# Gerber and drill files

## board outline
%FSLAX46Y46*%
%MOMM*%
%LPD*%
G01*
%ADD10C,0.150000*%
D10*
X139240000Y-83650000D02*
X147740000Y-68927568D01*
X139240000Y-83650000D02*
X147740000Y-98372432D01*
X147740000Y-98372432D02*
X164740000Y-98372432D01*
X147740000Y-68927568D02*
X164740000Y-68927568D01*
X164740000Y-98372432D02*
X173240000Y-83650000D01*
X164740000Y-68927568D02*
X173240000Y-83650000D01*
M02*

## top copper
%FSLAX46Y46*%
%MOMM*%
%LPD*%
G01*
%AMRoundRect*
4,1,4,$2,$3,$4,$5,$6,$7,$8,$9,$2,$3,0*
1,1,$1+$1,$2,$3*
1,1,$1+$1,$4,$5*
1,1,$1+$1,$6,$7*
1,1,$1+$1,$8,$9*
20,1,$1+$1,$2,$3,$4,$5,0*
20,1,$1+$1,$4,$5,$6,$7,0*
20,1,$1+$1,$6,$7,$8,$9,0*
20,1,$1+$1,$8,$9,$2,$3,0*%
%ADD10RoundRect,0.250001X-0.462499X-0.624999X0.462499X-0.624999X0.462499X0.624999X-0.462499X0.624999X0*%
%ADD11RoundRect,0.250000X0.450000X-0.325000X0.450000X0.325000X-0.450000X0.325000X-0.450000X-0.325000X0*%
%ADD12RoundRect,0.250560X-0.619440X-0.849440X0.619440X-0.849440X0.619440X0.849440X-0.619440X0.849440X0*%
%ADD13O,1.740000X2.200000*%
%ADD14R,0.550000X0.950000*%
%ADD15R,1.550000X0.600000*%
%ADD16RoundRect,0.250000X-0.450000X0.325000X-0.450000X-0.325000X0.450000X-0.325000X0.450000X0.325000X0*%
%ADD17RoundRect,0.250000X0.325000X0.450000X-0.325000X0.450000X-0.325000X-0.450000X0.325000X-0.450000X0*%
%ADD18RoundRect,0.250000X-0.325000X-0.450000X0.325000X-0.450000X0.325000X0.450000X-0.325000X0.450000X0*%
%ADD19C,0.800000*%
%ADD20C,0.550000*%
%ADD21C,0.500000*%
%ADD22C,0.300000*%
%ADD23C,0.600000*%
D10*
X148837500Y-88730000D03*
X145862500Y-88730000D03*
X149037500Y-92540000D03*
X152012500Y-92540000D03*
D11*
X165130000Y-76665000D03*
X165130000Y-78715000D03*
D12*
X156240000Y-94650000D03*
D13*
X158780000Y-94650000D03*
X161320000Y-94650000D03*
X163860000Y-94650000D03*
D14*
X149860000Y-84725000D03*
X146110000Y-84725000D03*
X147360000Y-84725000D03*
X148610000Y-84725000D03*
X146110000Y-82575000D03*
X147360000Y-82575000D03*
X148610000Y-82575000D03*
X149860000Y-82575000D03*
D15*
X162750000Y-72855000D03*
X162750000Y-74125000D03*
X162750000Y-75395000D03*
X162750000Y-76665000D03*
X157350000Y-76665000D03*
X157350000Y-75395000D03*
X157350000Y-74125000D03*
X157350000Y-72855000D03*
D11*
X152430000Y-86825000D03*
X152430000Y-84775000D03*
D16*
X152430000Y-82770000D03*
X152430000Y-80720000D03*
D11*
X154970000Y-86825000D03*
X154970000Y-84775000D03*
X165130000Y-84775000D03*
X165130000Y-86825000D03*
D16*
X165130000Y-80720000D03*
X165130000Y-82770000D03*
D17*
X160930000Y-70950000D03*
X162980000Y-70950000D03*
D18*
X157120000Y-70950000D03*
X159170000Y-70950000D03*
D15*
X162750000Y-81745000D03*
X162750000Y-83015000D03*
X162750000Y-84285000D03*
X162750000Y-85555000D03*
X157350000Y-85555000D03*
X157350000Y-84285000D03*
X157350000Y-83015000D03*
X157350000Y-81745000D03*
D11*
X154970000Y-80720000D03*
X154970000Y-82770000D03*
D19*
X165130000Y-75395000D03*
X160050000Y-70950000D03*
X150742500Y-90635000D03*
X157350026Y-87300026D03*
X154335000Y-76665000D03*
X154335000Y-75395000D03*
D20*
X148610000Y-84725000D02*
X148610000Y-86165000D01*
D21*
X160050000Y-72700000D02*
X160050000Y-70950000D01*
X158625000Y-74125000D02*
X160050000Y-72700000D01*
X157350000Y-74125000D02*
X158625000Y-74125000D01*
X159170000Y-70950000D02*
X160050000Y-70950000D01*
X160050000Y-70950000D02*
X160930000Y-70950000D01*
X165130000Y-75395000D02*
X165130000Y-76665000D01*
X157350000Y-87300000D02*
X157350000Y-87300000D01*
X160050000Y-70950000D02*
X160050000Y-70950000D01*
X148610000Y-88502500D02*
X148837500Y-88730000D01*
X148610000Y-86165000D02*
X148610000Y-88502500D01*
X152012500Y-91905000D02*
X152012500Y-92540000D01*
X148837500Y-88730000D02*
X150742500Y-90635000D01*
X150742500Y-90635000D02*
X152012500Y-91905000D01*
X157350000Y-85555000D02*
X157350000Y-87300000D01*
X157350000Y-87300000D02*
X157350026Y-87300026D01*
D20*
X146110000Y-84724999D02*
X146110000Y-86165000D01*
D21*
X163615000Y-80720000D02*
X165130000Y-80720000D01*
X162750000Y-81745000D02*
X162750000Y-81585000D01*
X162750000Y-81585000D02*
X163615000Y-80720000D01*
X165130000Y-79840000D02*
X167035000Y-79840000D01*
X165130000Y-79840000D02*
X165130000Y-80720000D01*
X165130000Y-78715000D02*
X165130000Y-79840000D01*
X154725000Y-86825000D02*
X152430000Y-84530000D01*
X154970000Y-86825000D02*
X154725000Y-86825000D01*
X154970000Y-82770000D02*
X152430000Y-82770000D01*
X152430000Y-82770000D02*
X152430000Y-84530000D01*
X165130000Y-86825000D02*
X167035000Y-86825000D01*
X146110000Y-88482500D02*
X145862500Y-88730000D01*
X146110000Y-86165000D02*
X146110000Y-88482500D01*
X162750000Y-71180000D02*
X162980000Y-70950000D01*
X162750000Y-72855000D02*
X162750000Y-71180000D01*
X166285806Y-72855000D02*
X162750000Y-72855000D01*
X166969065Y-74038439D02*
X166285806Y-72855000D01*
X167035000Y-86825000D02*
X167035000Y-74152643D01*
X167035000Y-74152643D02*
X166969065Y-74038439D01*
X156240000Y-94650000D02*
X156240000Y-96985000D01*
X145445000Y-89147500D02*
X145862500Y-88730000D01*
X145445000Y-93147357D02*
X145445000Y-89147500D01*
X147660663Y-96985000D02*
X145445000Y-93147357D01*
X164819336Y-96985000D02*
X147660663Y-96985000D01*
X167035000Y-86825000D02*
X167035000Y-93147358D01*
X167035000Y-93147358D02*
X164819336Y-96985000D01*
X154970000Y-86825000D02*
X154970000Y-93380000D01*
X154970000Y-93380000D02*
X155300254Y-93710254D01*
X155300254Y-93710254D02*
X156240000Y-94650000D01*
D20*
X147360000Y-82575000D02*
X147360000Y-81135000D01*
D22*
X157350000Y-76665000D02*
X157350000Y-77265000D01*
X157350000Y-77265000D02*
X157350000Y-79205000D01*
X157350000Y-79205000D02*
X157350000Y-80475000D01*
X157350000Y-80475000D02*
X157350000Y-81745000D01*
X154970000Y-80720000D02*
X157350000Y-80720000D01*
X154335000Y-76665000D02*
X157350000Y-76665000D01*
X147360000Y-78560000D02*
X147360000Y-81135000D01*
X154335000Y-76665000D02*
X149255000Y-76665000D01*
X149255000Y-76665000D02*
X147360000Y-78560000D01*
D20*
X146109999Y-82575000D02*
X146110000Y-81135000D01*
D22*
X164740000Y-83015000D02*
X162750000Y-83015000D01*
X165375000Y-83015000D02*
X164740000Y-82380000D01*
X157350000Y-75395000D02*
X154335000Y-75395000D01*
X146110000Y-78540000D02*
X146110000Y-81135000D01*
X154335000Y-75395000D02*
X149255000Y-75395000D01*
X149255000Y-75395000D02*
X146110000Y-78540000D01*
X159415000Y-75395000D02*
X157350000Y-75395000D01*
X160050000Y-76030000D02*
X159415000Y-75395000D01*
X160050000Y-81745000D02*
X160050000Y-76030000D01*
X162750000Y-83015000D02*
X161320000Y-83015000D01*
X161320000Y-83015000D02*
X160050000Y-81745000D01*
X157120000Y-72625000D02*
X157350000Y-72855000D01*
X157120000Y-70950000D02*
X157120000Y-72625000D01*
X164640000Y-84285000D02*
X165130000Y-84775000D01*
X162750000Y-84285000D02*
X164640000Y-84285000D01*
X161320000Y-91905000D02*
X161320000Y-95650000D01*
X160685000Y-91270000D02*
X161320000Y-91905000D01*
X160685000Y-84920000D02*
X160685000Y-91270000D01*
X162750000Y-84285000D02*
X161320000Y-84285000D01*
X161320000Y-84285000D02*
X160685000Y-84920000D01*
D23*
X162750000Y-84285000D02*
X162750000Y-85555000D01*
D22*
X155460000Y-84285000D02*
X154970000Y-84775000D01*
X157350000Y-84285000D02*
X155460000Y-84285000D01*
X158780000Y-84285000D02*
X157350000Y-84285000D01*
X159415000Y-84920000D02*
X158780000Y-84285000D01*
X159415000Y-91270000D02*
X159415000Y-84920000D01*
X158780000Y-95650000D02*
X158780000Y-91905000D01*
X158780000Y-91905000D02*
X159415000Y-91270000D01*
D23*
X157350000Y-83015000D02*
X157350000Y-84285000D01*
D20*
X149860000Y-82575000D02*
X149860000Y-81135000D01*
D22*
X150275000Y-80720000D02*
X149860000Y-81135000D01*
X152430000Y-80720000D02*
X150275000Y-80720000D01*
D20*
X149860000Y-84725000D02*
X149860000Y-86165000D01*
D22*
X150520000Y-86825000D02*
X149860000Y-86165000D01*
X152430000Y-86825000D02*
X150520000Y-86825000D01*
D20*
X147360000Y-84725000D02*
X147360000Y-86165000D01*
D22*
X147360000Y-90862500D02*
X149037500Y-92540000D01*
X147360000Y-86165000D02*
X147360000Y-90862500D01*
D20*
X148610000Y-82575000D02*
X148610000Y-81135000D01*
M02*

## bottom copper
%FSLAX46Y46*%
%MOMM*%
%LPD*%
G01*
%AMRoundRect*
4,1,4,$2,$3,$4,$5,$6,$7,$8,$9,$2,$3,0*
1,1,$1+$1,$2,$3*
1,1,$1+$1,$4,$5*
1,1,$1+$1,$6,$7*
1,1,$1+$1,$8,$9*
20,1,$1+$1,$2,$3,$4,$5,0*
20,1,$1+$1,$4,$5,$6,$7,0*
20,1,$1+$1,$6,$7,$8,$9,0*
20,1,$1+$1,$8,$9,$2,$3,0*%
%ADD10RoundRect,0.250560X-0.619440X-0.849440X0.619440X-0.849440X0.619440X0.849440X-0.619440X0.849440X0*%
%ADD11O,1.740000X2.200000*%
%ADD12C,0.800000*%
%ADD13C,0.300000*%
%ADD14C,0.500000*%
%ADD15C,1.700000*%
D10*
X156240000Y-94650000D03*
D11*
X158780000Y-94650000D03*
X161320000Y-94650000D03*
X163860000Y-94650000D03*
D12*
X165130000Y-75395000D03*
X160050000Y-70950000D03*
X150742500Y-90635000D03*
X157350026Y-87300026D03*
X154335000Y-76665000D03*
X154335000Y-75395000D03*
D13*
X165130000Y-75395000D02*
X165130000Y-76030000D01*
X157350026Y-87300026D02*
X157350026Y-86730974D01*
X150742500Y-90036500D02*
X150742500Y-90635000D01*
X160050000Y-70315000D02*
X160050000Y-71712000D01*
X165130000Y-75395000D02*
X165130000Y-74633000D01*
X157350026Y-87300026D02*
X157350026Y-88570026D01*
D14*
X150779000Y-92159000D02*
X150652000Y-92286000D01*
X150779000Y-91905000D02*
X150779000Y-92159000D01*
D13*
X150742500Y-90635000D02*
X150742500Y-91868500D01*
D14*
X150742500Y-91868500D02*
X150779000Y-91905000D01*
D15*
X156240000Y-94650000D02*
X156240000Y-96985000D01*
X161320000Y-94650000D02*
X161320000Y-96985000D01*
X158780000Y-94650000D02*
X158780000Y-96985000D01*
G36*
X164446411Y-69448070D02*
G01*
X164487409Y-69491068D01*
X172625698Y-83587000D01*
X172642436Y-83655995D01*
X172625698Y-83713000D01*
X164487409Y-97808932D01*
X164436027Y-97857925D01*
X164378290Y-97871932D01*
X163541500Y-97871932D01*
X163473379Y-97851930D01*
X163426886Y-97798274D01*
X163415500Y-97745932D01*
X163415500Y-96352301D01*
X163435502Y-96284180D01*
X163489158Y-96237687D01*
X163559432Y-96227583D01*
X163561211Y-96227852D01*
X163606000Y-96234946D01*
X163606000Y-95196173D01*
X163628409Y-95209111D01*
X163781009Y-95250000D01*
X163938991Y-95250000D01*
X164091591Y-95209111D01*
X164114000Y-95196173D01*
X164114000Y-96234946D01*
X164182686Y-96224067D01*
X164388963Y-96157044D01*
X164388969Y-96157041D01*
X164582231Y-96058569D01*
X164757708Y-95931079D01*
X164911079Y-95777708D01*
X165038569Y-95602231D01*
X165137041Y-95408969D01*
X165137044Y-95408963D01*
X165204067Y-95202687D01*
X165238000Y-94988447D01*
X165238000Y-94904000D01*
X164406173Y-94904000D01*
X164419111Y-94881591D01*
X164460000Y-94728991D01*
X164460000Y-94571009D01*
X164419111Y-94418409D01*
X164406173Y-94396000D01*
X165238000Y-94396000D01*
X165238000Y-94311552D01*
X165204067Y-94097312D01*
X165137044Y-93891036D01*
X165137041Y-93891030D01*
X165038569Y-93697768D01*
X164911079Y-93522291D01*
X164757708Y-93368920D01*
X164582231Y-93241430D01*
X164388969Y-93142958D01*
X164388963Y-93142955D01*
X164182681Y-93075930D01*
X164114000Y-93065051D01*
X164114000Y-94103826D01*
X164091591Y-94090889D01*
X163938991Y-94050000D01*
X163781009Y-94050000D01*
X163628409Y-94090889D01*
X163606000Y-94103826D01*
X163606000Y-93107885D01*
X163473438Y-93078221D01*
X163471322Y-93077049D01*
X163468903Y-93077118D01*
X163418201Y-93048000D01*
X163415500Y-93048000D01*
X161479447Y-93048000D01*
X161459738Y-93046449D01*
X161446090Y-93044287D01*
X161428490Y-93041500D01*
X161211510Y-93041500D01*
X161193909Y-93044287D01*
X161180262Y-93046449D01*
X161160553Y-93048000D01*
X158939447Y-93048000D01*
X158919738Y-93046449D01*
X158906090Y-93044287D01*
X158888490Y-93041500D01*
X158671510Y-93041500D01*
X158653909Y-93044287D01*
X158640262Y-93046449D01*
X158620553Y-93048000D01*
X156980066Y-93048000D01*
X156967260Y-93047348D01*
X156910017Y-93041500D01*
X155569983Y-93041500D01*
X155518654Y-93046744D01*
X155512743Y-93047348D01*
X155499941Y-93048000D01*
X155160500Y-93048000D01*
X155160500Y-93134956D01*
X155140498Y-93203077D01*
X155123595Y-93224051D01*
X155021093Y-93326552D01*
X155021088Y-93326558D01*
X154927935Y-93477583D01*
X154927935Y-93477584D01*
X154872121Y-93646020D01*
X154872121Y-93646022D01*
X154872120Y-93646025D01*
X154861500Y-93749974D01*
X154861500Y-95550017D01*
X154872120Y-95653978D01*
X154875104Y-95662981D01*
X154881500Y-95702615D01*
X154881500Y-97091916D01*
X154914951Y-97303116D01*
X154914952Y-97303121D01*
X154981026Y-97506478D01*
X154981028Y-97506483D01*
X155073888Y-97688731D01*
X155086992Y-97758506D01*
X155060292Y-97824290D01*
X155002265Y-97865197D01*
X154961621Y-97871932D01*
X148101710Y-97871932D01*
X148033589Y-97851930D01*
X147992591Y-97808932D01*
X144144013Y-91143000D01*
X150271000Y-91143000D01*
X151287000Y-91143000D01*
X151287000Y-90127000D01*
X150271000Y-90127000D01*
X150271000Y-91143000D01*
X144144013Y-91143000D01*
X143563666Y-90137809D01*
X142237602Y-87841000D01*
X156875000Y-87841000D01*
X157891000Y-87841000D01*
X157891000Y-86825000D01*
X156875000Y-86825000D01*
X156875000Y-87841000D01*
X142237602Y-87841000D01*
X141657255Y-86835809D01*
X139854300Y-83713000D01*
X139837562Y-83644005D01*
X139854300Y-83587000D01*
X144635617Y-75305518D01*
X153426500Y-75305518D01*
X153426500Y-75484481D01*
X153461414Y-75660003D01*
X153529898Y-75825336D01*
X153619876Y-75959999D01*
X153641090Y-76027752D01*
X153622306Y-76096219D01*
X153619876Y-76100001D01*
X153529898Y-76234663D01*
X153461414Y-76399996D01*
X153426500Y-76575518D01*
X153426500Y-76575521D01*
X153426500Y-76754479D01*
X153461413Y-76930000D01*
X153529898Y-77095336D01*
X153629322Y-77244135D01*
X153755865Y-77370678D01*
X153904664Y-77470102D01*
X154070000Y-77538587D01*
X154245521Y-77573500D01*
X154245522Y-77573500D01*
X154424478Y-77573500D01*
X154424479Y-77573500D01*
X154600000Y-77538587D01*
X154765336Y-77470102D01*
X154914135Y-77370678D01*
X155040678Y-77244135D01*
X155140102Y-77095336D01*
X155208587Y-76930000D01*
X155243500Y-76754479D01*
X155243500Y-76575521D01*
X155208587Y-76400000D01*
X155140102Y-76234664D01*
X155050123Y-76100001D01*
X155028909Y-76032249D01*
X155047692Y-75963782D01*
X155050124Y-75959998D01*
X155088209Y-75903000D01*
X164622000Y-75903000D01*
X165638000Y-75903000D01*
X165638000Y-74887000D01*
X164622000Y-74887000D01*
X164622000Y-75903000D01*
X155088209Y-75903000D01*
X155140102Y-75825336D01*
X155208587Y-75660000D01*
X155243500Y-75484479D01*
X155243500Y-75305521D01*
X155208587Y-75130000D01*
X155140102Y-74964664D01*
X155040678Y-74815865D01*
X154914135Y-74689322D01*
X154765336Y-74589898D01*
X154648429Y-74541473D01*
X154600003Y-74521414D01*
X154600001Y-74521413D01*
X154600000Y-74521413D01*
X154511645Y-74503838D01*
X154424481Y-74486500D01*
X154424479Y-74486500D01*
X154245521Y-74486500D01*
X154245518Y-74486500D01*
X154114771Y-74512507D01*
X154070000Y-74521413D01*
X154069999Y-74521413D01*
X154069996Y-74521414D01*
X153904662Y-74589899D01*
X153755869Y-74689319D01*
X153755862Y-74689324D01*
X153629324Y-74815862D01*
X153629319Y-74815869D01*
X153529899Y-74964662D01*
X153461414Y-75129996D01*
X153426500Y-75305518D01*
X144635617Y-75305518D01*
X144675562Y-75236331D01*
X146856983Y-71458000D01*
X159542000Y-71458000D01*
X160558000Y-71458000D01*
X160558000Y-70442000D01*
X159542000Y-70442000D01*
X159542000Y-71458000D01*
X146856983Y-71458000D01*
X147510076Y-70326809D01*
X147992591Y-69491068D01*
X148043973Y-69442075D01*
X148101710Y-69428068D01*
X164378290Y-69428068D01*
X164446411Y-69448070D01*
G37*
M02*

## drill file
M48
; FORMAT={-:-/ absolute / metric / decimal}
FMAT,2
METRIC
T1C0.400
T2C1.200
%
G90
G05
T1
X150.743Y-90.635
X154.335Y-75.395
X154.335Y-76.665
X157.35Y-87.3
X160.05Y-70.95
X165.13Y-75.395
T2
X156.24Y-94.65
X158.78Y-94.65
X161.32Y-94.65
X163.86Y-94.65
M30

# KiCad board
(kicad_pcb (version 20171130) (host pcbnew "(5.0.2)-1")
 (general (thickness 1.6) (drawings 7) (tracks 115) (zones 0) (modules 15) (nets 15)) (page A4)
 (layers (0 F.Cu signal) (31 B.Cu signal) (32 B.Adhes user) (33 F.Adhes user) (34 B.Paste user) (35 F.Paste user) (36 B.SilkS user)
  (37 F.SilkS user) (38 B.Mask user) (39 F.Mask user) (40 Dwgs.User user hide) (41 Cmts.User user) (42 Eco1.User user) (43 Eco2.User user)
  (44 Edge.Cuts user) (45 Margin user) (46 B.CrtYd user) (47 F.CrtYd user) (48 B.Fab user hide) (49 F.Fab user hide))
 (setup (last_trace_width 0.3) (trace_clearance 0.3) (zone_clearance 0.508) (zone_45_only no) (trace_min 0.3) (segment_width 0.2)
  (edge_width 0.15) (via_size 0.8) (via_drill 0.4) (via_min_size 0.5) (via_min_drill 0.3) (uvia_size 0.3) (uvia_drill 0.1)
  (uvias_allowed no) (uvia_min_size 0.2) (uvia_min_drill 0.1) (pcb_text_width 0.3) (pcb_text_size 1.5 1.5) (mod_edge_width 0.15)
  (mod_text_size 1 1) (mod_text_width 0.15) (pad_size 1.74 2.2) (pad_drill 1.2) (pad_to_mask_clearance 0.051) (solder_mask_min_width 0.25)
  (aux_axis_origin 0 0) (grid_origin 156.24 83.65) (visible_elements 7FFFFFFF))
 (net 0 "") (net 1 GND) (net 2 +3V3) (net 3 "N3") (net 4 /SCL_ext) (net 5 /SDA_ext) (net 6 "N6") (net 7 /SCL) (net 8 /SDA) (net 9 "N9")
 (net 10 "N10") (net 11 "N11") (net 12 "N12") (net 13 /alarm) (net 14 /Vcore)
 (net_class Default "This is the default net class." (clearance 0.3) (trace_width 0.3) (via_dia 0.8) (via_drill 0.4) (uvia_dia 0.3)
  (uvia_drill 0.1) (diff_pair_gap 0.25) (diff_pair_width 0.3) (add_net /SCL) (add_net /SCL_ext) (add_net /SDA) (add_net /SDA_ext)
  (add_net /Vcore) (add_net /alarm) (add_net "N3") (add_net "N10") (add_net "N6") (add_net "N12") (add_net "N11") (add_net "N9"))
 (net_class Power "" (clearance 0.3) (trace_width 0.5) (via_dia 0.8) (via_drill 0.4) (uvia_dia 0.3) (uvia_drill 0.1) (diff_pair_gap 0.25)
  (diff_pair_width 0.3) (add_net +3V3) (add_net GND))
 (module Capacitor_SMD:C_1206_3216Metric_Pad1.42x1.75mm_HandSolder (layer F.Cu) (at 147.35 88.73)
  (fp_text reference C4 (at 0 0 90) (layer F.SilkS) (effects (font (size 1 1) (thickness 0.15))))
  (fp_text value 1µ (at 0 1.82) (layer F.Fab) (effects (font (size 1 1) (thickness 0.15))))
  (pad 2 smd roundrect (at 1.4875 0) (size 1.425 1.75) (layers F.Cu F.Paste F.Mask) (roundrect_rratio 0.175439) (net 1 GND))
  (pad 1 smd roundrect (at -1.4875 0) (size 1.425 1.75) (layers F.Cu F.Paste F.Mask) (roundrect_rratio 0.175439) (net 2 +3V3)))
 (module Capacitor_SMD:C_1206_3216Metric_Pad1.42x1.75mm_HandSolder (layer F.Cu) (at 150.525 92.54)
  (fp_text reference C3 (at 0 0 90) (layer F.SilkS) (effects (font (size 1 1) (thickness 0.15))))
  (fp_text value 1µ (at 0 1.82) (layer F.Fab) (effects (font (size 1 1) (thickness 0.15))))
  (pad 1 smd roundrect (at -1.4875 0) (size 1.425 1.75) (layers F.Cu F.Paste F.Mask) (roundrect_rratio 0.175439) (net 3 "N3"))
  (pad 2 smd roundrect (at 1.4875 0) (size 1.425 1.75) (layers F.Cu F.Paste F.Mask) (roundrect_rratio 0.175439) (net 1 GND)))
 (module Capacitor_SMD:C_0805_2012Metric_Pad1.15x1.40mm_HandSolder (layer F.Cu) (at 165.13 77.69 90)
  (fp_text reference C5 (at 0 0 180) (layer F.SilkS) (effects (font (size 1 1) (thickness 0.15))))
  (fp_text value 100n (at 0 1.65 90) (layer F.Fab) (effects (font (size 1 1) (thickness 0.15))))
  (pad 2 smd roundrect (at 1.025 0 90) (size 1.15 1.4) (layers F.Cu F.Paste F.Mask) (roundrect_rratio 0.217391) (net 1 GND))
  (pad 1 smd roundrect (at -1.025 0 90) (size 1.15 1.4) (layers F.Cu F.Paste F.Mask) (roundrect_rratio 0.217391) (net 2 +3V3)))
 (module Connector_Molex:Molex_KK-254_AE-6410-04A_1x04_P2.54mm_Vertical (layer F.Cu) (at 156.24 94.65)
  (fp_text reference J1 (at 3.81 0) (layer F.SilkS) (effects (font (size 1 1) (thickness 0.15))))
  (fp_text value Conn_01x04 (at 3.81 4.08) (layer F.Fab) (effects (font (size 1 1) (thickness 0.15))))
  (pad 1 thru_hole roundrect (at 0 0) (size 1.74 2.2) (drill 1.2) (layers *.Cu *.Mask) (roundrect_rratio 0.144) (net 2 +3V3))
  (pad 2 thru_hole oval (at 2.54 0) (size 1.74 2.2) (drill 1.2) (layers *.Cu *.Mask) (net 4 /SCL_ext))
  (pad 3 thru_hole oval (at 5.08 0) (size 1.74 2.2) (drill 1.2) (layers *.Cu *.Mask) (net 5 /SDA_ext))
  (pad 4 thru_hole oval (at 7.62 0) (size 1.74 2.2) (drill 1.2) (layers *.Cu *.Mask) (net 1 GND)))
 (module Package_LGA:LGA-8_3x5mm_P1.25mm (layer F.Cu) (at 147.985 83.65 90)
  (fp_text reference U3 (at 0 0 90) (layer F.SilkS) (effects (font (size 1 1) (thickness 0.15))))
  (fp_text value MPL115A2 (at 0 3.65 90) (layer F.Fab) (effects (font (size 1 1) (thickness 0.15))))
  (pad 4 smd rect (at -1.075 1.875 90) (size 0.95 0.55) (layers F.Cu F.Paste F.Mask) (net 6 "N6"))
  (pad 1 smd rect (at -1.075 -1.875 90) (size 0.95 0.55) (layers F.Cu F.Paste F.Mask) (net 2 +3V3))
  (pad 2 smd rect (at -1.075 -0.625 90) (size 0.95 0.55) (layers F.Cu F.Paste F.Mask) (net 3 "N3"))
  (pad 3 smd rect (at -1.075 0.625 90) (size 0.95 0.55) (layers F.Cu F.Paste F.Mask) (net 1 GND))
  (pad 8 smd rect (at 1.075 -1.875 90) (size 0.95 0.55) (layers F.Cu F.Paste F.Mask) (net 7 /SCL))
  (pad 7 smd rect (at 1.075 -0.625 90) (size 0.95 0.55) (layers F.Cu F.Paste F.Mask) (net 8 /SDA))
  (pad 6 smd rect (at 1.075 0.625 90) (size 0.95 0.55) (layers F.Cu F.Paste F.Mask) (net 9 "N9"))
  (pad 5 smd rect (at 1.075 1.875 90) (size 0.95 0.55) (layers F.Cu F.Paste F.Mask) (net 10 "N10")))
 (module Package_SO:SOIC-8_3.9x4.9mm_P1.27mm (layer F.Cu) (at 160.05 74.76)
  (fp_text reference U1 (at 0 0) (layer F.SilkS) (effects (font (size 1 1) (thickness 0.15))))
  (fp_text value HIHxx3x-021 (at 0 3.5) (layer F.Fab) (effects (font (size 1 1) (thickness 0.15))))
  (pad 8 smd rect (at 2.7 -1.905) (size 1.55 0.6) (layers F.Cu F.Paste F.Mask) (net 2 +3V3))
  (pad 7 smd rect (at 2.7 -0.635) (size 1.55 0.6) (layers F.Cu F.Paste F.Mask) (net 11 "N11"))
  (pad 6 smd rect (at 2.7 0.635) (size 1.55 0.6) (layers F.Cu F.Paste F.Mask) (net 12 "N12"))
  (pad 5 smd rect (at 2.7 1.905) (size 1.55 0.6) (layers F.Cu F.Paste F.Mask) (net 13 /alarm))
  (pad 4 smd rect (at -2.7 1.905) (size 1.55 0.6) (layers F.Cu F.Paste F.Mask) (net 8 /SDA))
  (pad 3 smd rect (at -2.7 0.635) (size 1.55 0.6) (layers F.Cu F.Paste F.Mask) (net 7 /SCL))
  (pad 2 smd rect (at -2.7 -0.635) (size 1.55 0.6) (layers F.Cu F.Paste F.Mask) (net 1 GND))
  (pad 1 smd rect (at -2.7 -1.905) (size 1.55 0.6) (layers F.Cu F.Paste F.Mask) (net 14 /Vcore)))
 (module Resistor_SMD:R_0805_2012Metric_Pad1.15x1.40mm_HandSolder (layer F.Cu) (at 152.43 85.8 90)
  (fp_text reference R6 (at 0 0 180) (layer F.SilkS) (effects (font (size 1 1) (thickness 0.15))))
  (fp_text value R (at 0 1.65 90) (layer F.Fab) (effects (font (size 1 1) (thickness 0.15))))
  (pad 1 smd roundrect (at -1.025 0 90) (size 1.15 1.4) (layers F.Cu F.Paste F.Mask) (roundrect_rratio 0.217391) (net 6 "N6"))
  (pad 2 smd roundrect (at 1.025 0 90) (size 1.15 1.4) (layers F.Cu F.Paste F.Mask) (roundrect_rratio 0.217391) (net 2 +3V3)))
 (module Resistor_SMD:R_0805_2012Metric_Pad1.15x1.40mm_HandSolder (layer F.Cu) (at 152.43 81.745 270)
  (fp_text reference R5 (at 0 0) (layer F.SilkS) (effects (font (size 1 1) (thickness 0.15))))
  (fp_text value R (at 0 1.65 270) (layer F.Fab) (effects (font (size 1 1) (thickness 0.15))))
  (pad 2 smd roundrect (at 1.025 0 270) (size 1.15 1.4) (layers F.Cu F.Paste F.Mask) (roundrect_rratio 0.217391) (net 2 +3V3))
  (pad 1 smd roundrect (at -1.025 0 270) (size 1.15 1.4) (layers F.Cu F.Paste F.Mask) (roundrect_rratio 0.217391) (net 10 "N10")))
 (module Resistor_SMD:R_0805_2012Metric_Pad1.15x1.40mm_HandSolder (layer F.Cu) (at 154.97 85.8 90)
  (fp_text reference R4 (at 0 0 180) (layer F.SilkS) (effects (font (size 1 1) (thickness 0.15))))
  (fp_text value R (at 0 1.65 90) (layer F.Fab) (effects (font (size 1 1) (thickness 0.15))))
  (pad 1 smd roundrect (at -1.025 0 90) (size 1.15 1.4) (layers F.Cu F.Paste F.Mask) (roundrect_rratio 0.217391) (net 2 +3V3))
  (pad 2 smd roundrect (at 1.025 0 90) (size 1.15 1.4) (layers F.Cu F.Paste F.Mask) (roundrect_rratio 0.217391) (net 4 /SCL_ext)))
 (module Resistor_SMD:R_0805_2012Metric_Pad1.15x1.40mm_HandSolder (layer F.Cu) (at 165.13 85.8 90)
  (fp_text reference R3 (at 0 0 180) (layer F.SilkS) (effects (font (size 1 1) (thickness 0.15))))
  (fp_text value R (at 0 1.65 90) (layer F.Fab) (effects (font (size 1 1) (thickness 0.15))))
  (pad 2 smd roundrect (at 1.025 0 90) (size 1.15 1.4) (layers F.Cu F.Paste F.Mask) (roundrect_rratio 0.217391) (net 5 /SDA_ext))
  (pad 1 smd roundrect (at -1.025 0 90) (size 1.15 1.4) (layers F.Cu F.Paste F.Mask) (roundrect_rratio 0.217391) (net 2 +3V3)))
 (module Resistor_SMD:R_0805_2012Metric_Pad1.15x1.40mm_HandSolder (layer F.Cu) (at 165.13 81.745 270)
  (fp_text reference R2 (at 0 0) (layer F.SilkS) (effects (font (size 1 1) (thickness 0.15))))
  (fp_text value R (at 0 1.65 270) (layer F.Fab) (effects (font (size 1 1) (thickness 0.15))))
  (pad 1 smd roundrect (at -1.025 0 270) (size 1.15 1.4) (layers F.Cu F.Paste F.Mask) (roundrect_rratio 0.217391) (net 2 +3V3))
  (pad 2 smd roundrect (at 1.025 0 270) (size 1.15 1.4) (layers F.Cu F.Paste F.Mask) (roundrect_rratio 0.217391) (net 7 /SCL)))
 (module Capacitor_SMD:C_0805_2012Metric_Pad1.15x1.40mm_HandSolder (layer F.Cu) (at 161.955 70.95 180)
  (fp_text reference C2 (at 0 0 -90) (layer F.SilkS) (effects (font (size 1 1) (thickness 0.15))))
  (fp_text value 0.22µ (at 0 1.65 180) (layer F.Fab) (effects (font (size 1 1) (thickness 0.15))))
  (pad 2 smd roundrect (at 1.025 0 180) (size 1.15 1.4) (layers F.Cu F.Paste F.Mask) (roundrect_rratio 0.217391) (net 1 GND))
  (pad 1 smd roundrect (at -1.025 0 180) (size 1.15 1.4) (layers F.Cu F.Paste F.Mask) (roundrect_rratio 0.217391) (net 2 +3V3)))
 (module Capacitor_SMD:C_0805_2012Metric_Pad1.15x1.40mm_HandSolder (layer F.Cu) (at 158.145 70.95)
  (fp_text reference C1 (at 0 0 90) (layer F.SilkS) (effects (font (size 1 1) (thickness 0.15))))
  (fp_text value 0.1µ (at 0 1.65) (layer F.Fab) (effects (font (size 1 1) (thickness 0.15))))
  (pad 1 smd roundrect (at -1.025 0) (size 1.15 1.4) (layers F.Cu F.Paste F.Mask) (roundrect_rratio 0.217391) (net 14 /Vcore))
  (pad 2 smd roundrect (at 1.025 0) (size 1.15 1.4) (layers F.Cu F.Paste F.Mask) (roundrect_rratio 0.217391) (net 1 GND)))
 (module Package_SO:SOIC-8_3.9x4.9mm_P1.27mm (layer F.Cu) (at 160.05 83.65)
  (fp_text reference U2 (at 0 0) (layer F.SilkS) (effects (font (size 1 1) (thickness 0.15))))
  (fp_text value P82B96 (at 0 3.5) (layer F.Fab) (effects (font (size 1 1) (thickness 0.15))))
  (pad 8 smd rect (at 2.7 -1.905) (size 1.55 0.6) (layers F.Cu F.Paste F.Mask) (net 2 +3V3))
  (pad 7 smd rect (at 2.7 -0.635) (size 1.55 0.6) (layers F.Cu F.Paste F.Mask) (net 7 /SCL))
  (pad 6 smd rect (at 2.7 0.635) (size 1.55 0.6) (layers F.Cu F.Paste F.Mask) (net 5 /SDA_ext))
  (pad 5 smd rect (at 2.7 1.905) (size 1.55 0.6) (layers F.Cu F.Paste F.Mask) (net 5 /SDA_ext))
  (pad 4 smd rect (at -2.7 1.905) (size 1.55 0.6) (layers F.Cu F.Paste F.Mask) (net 1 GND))
  (pad 3 smd rect (at -2.7 0.635) (size 1.55 0.6) (layers F.Cu F.Paste F.Mask) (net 4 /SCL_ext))
  (pad 2 smd rect (at -2.7 -0.635) (size 1.55 0.6) (layers F.Cu F.Paste F.Mask) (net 4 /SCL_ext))
  (pad 1 smd rect (at -2.7 -1.905) (size 1.55 0.6) (layers F.Cu F.Paste F.Mask) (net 8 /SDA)))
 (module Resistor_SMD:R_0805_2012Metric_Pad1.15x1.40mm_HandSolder (layer F.Cu) (at 154.97 81.745 90)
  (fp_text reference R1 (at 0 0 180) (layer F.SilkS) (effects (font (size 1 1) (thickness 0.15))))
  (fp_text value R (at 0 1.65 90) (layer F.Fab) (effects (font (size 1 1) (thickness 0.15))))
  (pad 2 smd roundrect (at 1.025 0 90) (size 1.15 1.4) (layers F.Cu F.Paste F.Mask) (roundrect_rratio 0.217391) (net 8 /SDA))
  (pad 1 smd roundrect (at -1.025 0 90) (size 1.15 1.4) (layers F.Cu F.Paste F.Mask) (roundrect_rratio 0.217391) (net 2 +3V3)))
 (gr_line (start 139.24 83.65) (end 147.74 68.927568) (layer Edge.Cuts) (width 0.15))
 (gr_line (start 139.24 83.65) (end 147.74 98.372432) (layer Edge.Cuts) (width 0.15))
 (gr_line (start 147.74 98.372432) (end 164.74 98.372432) (layer Edge.Cuts) (width 0.15))
 (gr_line (start 147.74 68.927568) (end 164.74 68.927568) (layer Edge.Cuts) (width 0.15))
 (gr_line (start 164.74 98.372432) (end 173.24 83.65) (layer Edge.Cuts) (width 0.15))
 (gr_line (start 164.74 68.927568) (end 173.24 83.65) (layer Edge.Cuts) (width 0.15))
 (segment (start 148.61 84.725) (end 148.61 86.165) (width 0.55) (layer F.Cu) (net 1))
 (segment (start 160.05 72.7) (end 160.05 70.95) (width 0.5) (layer F.Cu) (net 1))
 (segment (start 158.625 74.125) (end 160.05 72.7) (width 0.5) (layer F.Cu) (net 1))
 (segment (start 157.35 74.125) (end 158.625 74.125) (width 0.5) (layer F.Cu) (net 1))
 (segment (start 159.17 70.95) (end 160.05 70.95) (width 0.5) (layer F.Cu) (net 1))
 (segment (start 160.05 70.95) (end 160.93 70.95) (width 0.5) (layer F.Cu) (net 1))
 (via (at 165.13 75.395) (size 0.8) (drill 0.4) (layers F.Cu B.Cu) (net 1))
 (segment (start 165.13 75.395) (end 165.13 76.665) (width 0.5) (layer F.Cu) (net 1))
 (segment (start 157.35 87.3) (end 157.35 87.3) (width 0.5) (layer F.Cu) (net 1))
 (segment (start 160.05 70.95) (end 160.05 70.95) (width 0.5) (layer F.Cu) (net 1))
 (via (at 160.05 70.95) (size 0.8) (drill 0.4) (layers F.Cu B.Cu) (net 1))
 (segment (start 148.61 88.5025) (end 148.8375 88.73) (width 0.5) (layer F.Cu) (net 1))
 (segment (start 148.61 86.165) (end 148.61 88.5025) (width 0.5) (layer F.Cu) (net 1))
 (segment (start 152.0125 91.905) (end 152.0125 92.54) (width 0.5) (layer F.Cu) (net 1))
 (segment (start 148.8375 88.73) (end 150.7425 90.635) (width 0.5) (layer F.Cu) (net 1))
 (segment (start 150.7425 90.635) (end 152.0125 91.905) (width 0.5) (layer F.Cu) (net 1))
 (via (at 150.7425 90.635) (size 0.8) (drill 0.4) (layers F.Cu B.Cu) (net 1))
 (segment (start 157.35 85.555) (end 157.35 87.3) (width 0.5) (layer F.Cu) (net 1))
 (segment (start 157.35 87.3) (end 157.350026 87.300026) (width 0.5) (layer F.Cu) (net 1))
 (via (at 157.350026 87.300026) (size 0.8) (drill 0.4) (layers F.Cu B.Cu) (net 1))
 (segment (start 165.13 75.395) (end 165.13 76.03) (width 0.3) (layer B.Cu) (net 1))
 (segment (start 157.350026 87.300026) (end 157.350026 86.730974) (width 0.3) (layer B.Cu) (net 1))
 (segment (start 150.7425 90.0365) (end 150.7425 90.635) (width 0.3) (layer B.Cu) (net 1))
 (segment (start 160.05 70.315) (end 160.05 71.712) (width 0.3) (layer B.Cu) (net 1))
 (segment (start 165.13 75.395) (end 165.13 74.633) (width 0.3) (layer B.Cu) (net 1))
 (segment (start 157.350026 87.300026) (end 157.350026 88.570026) (width 0.3) (layer B.Cu) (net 1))
 (segment (start 150.779 92.159) (end 150.652 92.286) (width 0.5) (layer B.Cu) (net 1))
 (segment (start 150.779 91.905) (end 150.779 92.159) (width 0.5) (layer B.Cu) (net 1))
 (segment (start 150.7425 90.635) (end 150.7425 91.8685) (width 0.3) (layer B.Cu) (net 1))
 (segment (start 150.7425 91.8685) (end 150.779 91.905) (width 0.5) (layer B.Cu) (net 1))
 (segment (start 146.11 84.724999) (end 146.11 86.165) (width 0.55) (layer F.Cu) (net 2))
 (segment (start 163.615 80.72) (end 165.13 80.72) (width 0.5) (layer F.Cu) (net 2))
 (segment (start 162.75 81.745) (end 162.75 81.585) (width 0.5) (layer F.Cu) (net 2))
 (segment (start 162.75 81.585) (end 163.615 80.72) (width 0.5) (layer F.Cu) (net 2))
 (segment (start 165.13 79.84) (end 167.035 79.84) (width 0.5) (layer F.Cu) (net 2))
 (segment (start 165.13 79.84) (end 165.13 80.72) (width 0.5) (layer F.Cu) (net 2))
 (segment (start 165.13 78.715) (end 165.13 79.84) (width 0.5) (layer F.Cu) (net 2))
 (segment (start 154.725 86.825) (end 152.43 84.53) (width 0.5) (layer F.Cu) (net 2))
 (segment (start 154.97 86.825) (end 154.725 86.825) (width 0.5) (layer F.Cu) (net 2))
 (segment (start 154.97 82.77) (end 152.43 82.77) (width 0.5) (layer F.Cu) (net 2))
 (segment (start 152.43 82.77) (end 152.43 84.53) (width 0.5) (layer F.Cu) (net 2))
 (segment (start 165.13 86.825) (end 167.035 86.825) (width 0.5) (layer F.Cu) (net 2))
 (segment (start 146.11 88.4825) (end 145.8625 88.73) (width 0.5) (layer F.Cu) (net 2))
 (segment (start 146.11 86.165) (end 146.11 88.4825) (width 0.5) (layer F.Cu) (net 2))
 (segment (start 162.75 71.18) (end 162.98 70.95) (width 0.5) (layer F.Cu) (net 2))
 (segment (start 162.75 72.855) (end 162.75 71.18) (width 0.5) (layer F.Cu) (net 2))
 (segment (start 166.285806 72.855) (end 162.75 72.855) (width 0.5) (layer F.Cu) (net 2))
 (segment (start 166.969065 74.038439) (end 166.285806 72.855) (width 0.5) (layer F.Cu) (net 2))
 (segment (start 167.035 86.825) (end 167.035 74.152643) (width 0.5) (layer F.Cu) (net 2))
 (segment (start 167.035 74.152643) (end 166.969065 74.038439) (width 0.5) (layer F.Cu) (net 2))
 (segment (start 156.24 94.65) (end 156.24 96.985) (width 0.5) (layer F.Cu) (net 2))
 (segment (start 145.445 89.1475) (end 145.8625 88.73) (width 0.5) (layer F.Cu) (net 2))
 (segment (start 145.445 93.147357) (end 145.445 89.1475) (width 0.5) (layer F.Cu) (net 2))
 (segment (start 147.660663 96.985) (end 145.445 93.147357) (width 0.5) (layer F.Cu) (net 2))
 (segment (start 164.819336 96.985) (end 147.660663 96.985) (width 0.5) (layer F.Cu) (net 2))
 (segment (start 167.035 86.825) (end 167.035 93.147358) (width 0.5) (layer F.Cu) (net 2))
 (segment (start 167.035 93.147358) (end 164.819336 96.985) (width 0.5) (layer F.Cu) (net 2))
 (segment (start 156.24 94.65) (end 156.24 96.985) (width 1.7) (layer B.Cu) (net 2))
 (segment (start 154.97 86.825) (end 154.97 93.38) (width 0.5) (layer F.Cu) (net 2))
 (segment (start 154.97 93.38) (end 155.300254 93.710254) (width 0.5) (layer F.Cu) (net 2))
 (segment (start 155.300254 93.710254) (end 156.24 94.65) (width 0.5) (layer F.Cu) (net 2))
 (segment (start 147.36 82.575) (end 147.36 81.135) (width 0.55) (layer F.Cu) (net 8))
 (segment (start 157.35 76.665) (end 157.35 77.265) (width 0.3) (layer F.Cu) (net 8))
 (segment (start 157.35 77.265) (end 157.35 79.205) (width 0.3) (layer F.Cu) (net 8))
 (segment (start 157.35 79.205) (end 157.35 80.475) (width 0.3) (layer F.Cu) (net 8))
 (segment (start 157.35 80.475) (end 157.35 81.745) (width 0.3) (layer F.Cu) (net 8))
 (segment (start 154.97 80.72) (end 157.35 80.72) (width 0.3) (layer F.Cu) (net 8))
 (segment (start 154.335 76.665) (end 157.35 76.665) (width 0.3) (layer F.Cu) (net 8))
 (via (at 154.335 76.665) (size 0.8) (drill 0.4) (layers F.Cu B.Cu) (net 8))
 (segment (start 147.36 78.56) (end 147.36 81.135) (width 0.3) (layer F.Cu) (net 8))
 (segment (start 154.335 76.665) (end 149.255 76.665) (width 0.3) (layer F.Cu) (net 8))
 (segment (start 149.255 76.665) (end 147.36 78.56) (width 0.3) (layer F.Cu) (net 8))
 (segment (start 146.109999 82.575) (end 146.11 81.135) (width 0.55) (layer F.Cu) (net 7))
 (segment (start 164.74 83.015) (end 162.75 83.015) (width 0.3) (layer F.Cu) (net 7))
 (segment (start 165.375 83.015) (end 164.74 82.38) (width 0.3) (layer F.Cu) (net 7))
 (segment (start 157.35 75.395) (end 154.335 75.395) (width 0.3) (layer F.Cu) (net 7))
 (via (at 154.335 75.395) (size 0.8) (drill 0.4) (layers F.Cu B.Cu) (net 7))
 (segment (start 146.11 78.54) (end 146.11 81.135) (width 0.3) (layer F.Cu) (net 7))
 (segment (start 154.335 75.395) (end 149.255 75.395) (width 0.3) (layer F.Cu) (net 7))
 (segment (start 149.255 75.395) (end 146.11 78.54) (width 0.3) (layer F.Cu) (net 7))
 (segment (start 159.415 75.395) (end 157.35 75.395) (width 0.3) (layer F.Cu) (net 7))
 (segment (start 160.05 76.03) (end 159.415 75.395) (width 0.3) (layer F.Cu) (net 7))
 (segment (start 160.05 81.745) (end 160.05 76.03) (width 0.3) (layer F.Cu) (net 7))
 (segment (start 162.75 83.015) (end 161.32 83.015) (width 0.3) (layer F.Cu) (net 7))
 (segment (start 161.32 83.015) (end 160.05 81.745) (width 0.3) (layer F.Cu) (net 7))
 (segment (start 157.12 72.625) (end 157.35 72.855) (width 0.3) (layer F.Cu) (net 14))
 (segment (start 157.12 70.95) (end 157.12 72.625) (width 0.3) (layer F.Cu) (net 14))
 (segment (start 164.64 84.285) (end 165.13 84.775) (width 0.3) (layer F.Cu) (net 5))
 (segment (start 162.75 84.285) (end 164.64 84.285) (width 0.3) (layer F.Cu) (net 5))
 (segment (start 161.32 91.905) (end 161.32 95.65) (width 0.3) (layer F.Cu) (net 5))
 (segment (start 160.685 91.27) (end 161.32 91.905) (width 0.3) (layer F.Cu) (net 5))
 (segment (start 160.685 84.92) (end 160.685 91.27) (width 0.3) (layer F.Cu) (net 5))
 (segment (start 162.75 84.285) (end 161.32 84.285) (width 0.3) (layer F.Cu) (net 5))
 (segment (start 161.32 84.285) (end 160.685 84.92) (width 0.3) (layer F.Cu) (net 5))
 (segment (start 162.75 84.285) (end 162.75 85.555) (width 0.6) (layer F.Cu) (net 5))
 (segment (start 161.32 94.65) (end 161.32 96.985) (width 1.7) (layer B.Cu) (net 5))
 (segment (start 155.46 84.285) (end 154.97 84.775) (width 0.3) (layer F.Cu) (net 4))
 (segment (start 157.35 84.285) (end 155.46 84.285) (width 0.3) (layer F.Cu) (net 4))
 (segment (start 158.78 84.285) (end 157.35 84.285) (width 0.3) (layer F.Cu) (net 4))
 (segment (start 159.415 84.92) (end 158.78 84.285) (width 0.3) (layer F.Cu) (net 4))
 (segment (start 159.415 91.27) (end 159.415 84.92) (width 0.3) (layer F.Cu) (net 4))
 (segment (start 158.78 95.65) (end 158.78 91.905) (width 0.3) (layer F.Cu) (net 4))
 (segment (start 158.78 91.905) (end 159.415 91.27) (width 0.3) (layer F.Cu) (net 4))
 (segment (start 157.35 83.015) (end 157.35 84.285) (width 0.6) (layer F.Cu) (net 4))
 (segment (start 158.78 94.65) (end 158.78 96.985) (width 1.7) (layer B.Cu) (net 4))
 (segment (start 149.86 82.575) (end 149.86 81.135) (width 0.55) (layer F.Cu) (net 10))
 (segment (start 150.275 80.72) (end 149.86 81.135) (width 0.3) (layer F.Cu) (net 10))
 (segment (start 152.43 80.72) (end 150.275 80.72) (width 0.3) (layer F.Cu) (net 10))
 (segment (start 149.86 84.725) (end 149.86 86.165) (width 0.55) (layer F.Cu) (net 6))
 (segment (start 150.52 86.825) (end 149.86 86.165) (width 0.3) (layer F.Cu) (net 6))
 (segment (start 152.43 86.825) (end 150.52 86.825) (width 0.3) (layer F.Cu) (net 6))
 (segment (start 147.36 84.725) (end 147.36 86.165) (width 0.55) (layer F.Cu) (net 3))
 (segment (start 147.36 90.8625) (end 149.0375 92.54) (width 0.3) (layer F.Cu) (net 3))
 (segment (start 147.36 86.165) (end 147.36 90.8625) (width 0.3) (layer F.Cu) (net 3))
 (segment (start 148.61 82.575) (end 148.61 81.135) (width 0.55) (layer F.Cu) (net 9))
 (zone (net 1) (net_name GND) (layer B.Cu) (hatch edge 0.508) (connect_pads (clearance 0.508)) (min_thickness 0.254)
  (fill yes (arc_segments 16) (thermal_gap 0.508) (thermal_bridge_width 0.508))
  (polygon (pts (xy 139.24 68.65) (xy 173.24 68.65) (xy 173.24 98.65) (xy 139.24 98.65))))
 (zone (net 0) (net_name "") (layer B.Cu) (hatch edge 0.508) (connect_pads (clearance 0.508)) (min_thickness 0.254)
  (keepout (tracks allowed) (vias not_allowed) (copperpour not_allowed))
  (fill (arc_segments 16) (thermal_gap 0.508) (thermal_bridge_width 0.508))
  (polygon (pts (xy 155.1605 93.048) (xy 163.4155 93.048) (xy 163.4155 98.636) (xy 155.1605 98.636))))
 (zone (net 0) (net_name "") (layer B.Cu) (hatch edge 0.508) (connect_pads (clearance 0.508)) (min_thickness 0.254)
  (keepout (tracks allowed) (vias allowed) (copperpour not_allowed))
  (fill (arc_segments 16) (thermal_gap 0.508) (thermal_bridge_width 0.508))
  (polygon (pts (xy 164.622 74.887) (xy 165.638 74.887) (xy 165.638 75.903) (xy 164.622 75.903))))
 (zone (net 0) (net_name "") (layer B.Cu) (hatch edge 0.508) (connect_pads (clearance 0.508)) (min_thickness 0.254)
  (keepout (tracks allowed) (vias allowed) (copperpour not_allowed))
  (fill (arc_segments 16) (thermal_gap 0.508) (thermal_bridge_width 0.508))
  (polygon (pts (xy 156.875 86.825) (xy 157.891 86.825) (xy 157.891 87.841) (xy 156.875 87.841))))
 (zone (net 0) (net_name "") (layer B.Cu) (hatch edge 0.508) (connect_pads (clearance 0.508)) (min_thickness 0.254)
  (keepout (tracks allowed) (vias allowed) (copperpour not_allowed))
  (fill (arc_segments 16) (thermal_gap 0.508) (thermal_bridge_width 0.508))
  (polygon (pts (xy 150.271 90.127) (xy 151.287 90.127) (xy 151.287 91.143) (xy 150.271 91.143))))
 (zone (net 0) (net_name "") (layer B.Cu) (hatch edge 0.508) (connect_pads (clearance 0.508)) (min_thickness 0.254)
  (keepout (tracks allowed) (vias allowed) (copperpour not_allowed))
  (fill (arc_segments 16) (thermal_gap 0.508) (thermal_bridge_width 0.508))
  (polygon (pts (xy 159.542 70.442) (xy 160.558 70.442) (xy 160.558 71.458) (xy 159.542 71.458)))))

